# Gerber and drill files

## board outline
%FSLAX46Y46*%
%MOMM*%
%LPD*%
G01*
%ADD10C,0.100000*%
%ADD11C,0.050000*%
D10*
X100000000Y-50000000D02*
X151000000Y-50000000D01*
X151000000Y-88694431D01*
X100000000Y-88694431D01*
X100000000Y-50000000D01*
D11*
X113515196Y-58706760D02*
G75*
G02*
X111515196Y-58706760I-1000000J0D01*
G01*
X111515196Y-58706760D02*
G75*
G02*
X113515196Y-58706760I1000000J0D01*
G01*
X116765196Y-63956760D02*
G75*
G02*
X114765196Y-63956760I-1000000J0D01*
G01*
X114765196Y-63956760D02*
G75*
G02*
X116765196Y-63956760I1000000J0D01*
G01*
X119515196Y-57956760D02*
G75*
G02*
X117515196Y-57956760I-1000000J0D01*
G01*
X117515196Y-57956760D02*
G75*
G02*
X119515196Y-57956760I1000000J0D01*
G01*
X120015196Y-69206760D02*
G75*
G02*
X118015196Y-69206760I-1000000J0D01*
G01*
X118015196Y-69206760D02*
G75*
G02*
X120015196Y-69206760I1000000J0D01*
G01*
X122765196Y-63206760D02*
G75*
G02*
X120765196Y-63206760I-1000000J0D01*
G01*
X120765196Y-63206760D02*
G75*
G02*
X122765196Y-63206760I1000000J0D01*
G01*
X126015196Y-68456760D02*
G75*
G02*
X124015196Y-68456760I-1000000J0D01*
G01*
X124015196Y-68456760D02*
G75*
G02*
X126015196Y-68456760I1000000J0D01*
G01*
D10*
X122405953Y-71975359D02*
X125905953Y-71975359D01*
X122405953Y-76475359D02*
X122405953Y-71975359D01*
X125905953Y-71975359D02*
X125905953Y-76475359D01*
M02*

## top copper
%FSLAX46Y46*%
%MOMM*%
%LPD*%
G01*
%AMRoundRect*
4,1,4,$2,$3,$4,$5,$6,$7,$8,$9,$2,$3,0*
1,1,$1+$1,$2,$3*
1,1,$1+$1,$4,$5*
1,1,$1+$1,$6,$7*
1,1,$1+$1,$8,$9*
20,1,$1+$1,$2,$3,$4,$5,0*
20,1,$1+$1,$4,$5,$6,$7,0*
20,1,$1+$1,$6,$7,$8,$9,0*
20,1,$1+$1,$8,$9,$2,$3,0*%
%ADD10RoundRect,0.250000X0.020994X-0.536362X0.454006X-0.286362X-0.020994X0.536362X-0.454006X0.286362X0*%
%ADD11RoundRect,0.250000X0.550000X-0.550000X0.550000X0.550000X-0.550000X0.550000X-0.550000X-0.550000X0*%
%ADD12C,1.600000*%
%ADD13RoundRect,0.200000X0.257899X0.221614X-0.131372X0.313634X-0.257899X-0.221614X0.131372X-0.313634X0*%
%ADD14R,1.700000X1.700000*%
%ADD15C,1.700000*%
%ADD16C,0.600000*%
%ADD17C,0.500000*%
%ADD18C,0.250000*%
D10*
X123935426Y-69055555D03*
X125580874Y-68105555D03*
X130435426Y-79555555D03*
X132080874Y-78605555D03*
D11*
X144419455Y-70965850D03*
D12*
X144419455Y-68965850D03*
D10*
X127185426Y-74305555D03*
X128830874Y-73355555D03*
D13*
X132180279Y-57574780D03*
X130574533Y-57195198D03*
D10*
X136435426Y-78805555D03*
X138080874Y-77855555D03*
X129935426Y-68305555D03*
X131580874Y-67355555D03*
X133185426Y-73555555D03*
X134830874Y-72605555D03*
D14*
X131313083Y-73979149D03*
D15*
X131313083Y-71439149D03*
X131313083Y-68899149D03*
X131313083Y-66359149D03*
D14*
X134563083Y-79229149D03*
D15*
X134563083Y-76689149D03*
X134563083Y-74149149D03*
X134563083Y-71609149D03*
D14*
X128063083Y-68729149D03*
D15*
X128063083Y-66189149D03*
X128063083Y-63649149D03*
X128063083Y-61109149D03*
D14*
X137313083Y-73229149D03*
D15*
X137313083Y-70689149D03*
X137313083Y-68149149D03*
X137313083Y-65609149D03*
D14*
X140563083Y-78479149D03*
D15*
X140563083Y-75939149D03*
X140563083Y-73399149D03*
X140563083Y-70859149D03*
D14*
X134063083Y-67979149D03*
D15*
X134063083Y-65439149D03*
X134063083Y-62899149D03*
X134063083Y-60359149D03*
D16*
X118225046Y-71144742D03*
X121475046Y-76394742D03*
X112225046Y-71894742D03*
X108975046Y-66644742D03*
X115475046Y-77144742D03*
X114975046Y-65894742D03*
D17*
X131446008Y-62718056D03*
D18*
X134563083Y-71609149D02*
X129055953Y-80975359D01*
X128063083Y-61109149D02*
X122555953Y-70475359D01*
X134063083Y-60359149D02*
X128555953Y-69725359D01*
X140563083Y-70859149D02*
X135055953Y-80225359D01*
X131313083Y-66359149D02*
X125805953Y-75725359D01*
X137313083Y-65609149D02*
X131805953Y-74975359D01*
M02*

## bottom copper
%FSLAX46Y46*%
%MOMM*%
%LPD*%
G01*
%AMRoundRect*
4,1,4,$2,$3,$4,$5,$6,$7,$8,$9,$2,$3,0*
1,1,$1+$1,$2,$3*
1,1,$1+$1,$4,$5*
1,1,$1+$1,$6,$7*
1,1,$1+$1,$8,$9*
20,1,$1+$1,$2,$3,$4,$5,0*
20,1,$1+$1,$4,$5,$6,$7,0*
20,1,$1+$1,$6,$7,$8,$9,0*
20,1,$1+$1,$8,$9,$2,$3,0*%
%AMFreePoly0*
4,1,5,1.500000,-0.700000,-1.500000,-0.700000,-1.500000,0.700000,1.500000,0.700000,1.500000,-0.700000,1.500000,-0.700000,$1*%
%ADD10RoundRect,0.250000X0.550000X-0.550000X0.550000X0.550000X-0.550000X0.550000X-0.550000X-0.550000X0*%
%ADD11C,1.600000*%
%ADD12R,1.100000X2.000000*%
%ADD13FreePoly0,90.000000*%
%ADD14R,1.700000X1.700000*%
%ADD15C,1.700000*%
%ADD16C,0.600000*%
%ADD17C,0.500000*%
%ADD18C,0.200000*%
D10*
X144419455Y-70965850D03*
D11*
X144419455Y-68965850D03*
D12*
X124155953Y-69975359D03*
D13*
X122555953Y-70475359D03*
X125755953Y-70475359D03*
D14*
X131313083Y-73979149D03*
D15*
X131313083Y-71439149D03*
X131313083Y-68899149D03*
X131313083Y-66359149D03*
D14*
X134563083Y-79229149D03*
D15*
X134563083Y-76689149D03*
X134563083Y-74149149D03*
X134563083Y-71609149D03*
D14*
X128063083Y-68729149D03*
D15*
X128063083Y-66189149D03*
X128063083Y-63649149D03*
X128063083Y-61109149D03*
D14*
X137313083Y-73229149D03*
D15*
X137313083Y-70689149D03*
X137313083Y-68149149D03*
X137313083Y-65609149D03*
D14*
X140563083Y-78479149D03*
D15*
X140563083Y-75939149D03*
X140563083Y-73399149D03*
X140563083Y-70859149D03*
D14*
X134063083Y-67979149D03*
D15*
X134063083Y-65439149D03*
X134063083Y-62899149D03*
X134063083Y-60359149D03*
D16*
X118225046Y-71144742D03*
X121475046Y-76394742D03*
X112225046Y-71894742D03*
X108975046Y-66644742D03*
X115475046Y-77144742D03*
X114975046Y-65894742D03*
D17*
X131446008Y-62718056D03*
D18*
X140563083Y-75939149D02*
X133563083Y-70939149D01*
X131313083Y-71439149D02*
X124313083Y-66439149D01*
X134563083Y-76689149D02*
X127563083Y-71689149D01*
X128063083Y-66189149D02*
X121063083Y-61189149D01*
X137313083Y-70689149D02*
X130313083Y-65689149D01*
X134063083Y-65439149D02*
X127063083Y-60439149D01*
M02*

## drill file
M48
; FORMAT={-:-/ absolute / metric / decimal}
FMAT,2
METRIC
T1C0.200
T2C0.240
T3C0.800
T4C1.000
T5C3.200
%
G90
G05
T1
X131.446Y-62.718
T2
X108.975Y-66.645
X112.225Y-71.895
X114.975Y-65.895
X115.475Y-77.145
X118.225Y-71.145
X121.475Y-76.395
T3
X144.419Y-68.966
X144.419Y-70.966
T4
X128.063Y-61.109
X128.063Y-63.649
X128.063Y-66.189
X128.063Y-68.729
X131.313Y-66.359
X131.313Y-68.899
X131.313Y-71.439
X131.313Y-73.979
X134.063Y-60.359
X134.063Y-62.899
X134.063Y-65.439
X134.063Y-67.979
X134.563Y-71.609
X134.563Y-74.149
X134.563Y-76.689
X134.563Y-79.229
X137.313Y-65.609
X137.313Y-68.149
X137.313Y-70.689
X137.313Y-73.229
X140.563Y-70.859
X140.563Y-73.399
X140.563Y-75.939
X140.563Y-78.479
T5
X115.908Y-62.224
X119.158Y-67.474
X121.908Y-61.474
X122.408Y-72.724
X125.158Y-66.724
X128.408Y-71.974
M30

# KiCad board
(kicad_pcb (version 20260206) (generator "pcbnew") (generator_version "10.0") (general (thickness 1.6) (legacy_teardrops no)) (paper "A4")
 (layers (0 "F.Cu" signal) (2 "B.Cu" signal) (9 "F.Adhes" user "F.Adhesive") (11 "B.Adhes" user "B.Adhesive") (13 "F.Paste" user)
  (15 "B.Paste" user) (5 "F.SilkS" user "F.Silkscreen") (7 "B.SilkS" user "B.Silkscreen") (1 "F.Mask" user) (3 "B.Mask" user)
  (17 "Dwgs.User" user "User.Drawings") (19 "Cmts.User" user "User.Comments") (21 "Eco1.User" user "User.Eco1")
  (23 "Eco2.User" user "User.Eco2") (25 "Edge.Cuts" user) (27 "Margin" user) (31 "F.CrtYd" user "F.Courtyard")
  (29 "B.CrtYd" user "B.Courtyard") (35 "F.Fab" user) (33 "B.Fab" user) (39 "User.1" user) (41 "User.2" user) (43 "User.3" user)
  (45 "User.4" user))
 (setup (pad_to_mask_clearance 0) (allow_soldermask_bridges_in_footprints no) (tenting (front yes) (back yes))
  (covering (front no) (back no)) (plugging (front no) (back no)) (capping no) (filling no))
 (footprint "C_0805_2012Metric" (layer "F.Cu") (at 124.75815 68.580555 30)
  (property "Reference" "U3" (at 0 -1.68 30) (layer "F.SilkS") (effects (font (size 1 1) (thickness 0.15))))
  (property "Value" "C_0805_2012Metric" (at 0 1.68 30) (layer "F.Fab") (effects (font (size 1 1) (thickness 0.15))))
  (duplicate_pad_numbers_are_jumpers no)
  (pad "1" smd roundrect (at -0.95 0 30) (size 1 1.45) (layers "F.Cu" "F.Mask" "F.Paste") (roundrect_rratio 0.25) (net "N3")
   (clearance 0.35))
  (pad "2" smd roundrect (at 0.95 0 30) (size 1 1.45) (layers "F.Cu" "F.Mask" "F.Paste") (roundrect_rratio 0.25)))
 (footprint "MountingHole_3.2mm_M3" (layer "F.Cu") (at 119.158484 67.474067 45)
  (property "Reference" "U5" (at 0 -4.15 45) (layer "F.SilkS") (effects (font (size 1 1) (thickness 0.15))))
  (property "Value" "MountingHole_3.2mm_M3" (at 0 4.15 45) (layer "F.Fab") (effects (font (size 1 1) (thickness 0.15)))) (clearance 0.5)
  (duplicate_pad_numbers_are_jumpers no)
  (pad "" np_thru_hole circle (at 0 0 45) (size 3.2 3.2) (drill 3.2) (layers "*.Cu" "*.Mask")))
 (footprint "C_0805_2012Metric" (layer "F.Cu") (at 131.25815 79.080555 30)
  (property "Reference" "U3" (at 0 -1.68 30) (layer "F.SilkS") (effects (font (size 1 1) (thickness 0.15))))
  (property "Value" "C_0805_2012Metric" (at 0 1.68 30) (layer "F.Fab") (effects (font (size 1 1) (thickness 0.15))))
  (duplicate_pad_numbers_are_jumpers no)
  (pad "1" smd roundrect (at -0.95 0 30) (size 1 1.45) (layers "F.Cu" "F.Mask" "F.Paste") (roundrect_rratio 0.25) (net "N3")
   (clearance 0.35))
  (pad "2" smd roundrect (at 0.95 0 30) (size 1 1.45) (layers "F.Cu" "F.Mask" "F.Paste") (roundrect_rratio 0.25)))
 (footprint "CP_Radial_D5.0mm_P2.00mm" (layer "F.Cu") (at 144.419455 70.96585 90)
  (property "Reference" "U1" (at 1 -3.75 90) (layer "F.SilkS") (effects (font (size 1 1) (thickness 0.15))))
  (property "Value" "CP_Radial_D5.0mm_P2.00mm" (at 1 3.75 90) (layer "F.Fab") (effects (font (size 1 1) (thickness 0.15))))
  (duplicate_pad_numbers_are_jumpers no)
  (pad "1" thru_hole roundrect (at 0 0 90) (size 1.6 1.6) (drill 0.8) (layers "*.Cu" "*.Mask") (remove_unused_layers no)
   (roundrect_rratio 0.15625) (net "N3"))
  (pad "2" thru_hole circle (at 2 0 90) (size 1.6 1.6) (drill 0.8) (layers "*.Cu" "*.Mask") (remove_unused_layers no) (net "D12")))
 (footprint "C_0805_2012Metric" (layer "F.Cu") (at 128.00815 73.830555 30)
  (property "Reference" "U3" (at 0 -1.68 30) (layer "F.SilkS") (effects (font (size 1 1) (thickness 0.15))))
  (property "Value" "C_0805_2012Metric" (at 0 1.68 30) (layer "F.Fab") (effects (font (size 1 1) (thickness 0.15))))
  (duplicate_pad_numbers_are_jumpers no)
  (pad "1" smd roundrect (at -0.95 0 30) (size 1 1.45) (layers "F.Cu" "F.Mask" "F.Paste") (roundrect_rratio 0.25) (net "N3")
   (clearance 0.35))
  (pad "2" smd roundrect (at 0.95 0 30) (size 1 1.45) (layers "F.Cu" "F.Mask" "F.Paste") (roundrect_rratio 0.25)))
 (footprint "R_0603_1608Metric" (layer "F.Cu") (at 131.377406 57.384989 166.7)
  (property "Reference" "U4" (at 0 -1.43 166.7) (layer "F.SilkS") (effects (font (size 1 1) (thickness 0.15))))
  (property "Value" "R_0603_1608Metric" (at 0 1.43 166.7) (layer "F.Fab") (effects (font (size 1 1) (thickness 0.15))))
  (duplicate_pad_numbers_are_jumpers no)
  (pad "1" smd roundrect (at -0.825 0 166.7) (size 0.8 0.95) (layers "F.Cu" "F.Mask" "F.Paste") (roundrect_rratio 0.25) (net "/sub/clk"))
  (pad "2" smd roundrect (at 0.825 0 166.7) (size 0.8 0.95) (layers "F.Cu" "F.Mask" "F.Paste") (roundrect_rratio 0.25) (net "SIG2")))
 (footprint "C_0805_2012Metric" (layer "F.Cu") (at 137.25815 78.330555 30)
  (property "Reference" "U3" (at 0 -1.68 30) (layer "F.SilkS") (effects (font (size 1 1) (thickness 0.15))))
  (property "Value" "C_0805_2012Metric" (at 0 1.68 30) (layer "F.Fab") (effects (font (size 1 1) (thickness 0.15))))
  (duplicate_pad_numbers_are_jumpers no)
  (pad "1" smd roundrect (at -0.95 0 30) (size 1 1.45) (layers "F.Cu" "F.Mask" "F.Paste") (roundrect_rratio 0.25) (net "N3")
   (clearance 0.35))
  (pad "2" smd roundrect (at 0.95 0 30) (size 1 1.45) (layers "F.Cu" "F.Mask" "F.Paste") (roundrect_rratio 0.25)))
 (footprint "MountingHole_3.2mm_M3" (layer "F.Cu") (at 115.908484 62.224067 45)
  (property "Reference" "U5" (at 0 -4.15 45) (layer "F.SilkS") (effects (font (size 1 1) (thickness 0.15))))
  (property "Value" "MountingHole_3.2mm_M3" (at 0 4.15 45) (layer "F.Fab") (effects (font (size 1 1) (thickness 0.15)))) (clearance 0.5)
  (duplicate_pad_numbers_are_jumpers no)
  (pad "" np_thru_hole circle (at 0 0 45) (size 3.2 3.2) (drill 3.2) (layers "*.Cu" "*.Mask")))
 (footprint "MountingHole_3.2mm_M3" (layer "F.Cu") (at 122.408484 72.724067 45)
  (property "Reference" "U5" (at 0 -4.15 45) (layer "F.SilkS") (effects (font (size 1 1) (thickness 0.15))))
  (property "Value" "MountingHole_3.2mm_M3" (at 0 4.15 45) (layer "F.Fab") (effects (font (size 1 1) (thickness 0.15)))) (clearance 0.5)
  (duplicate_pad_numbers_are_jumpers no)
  (pad "" np_thru_hole circle (at 0 0 45) (size 3.2 3.2) (drill 3.2) (layers "*.Cu" "*.Mask")))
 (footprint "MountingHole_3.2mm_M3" (layer "F.Cu") (at 125.158484 66.724067 45)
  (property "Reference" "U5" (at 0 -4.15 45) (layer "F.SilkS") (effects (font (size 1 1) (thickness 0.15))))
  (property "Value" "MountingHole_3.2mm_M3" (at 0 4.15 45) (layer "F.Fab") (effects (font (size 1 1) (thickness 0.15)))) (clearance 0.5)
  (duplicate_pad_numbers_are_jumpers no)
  (pad "" np_thru_hole circle (at 0 0 45) (size 3.2 3.2) (drill 3.2) (layers "*.Cu" "*.Mask")))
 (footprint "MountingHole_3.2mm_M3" (layer "F.Cu") (at 121.908484 61.474067 45)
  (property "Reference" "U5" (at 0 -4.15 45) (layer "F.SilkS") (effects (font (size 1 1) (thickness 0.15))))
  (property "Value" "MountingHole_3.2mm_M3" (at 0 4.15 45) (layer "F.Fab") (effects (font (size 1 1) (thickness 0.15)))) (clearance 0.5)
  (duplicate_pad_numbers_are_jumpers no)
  (pad "" np_thru_hole circle (at 0 0 45) (size 3.2 3.2) (drill 3.2) (layers "*.Cu" "*.Mask")))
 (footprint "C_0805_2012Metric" (layer "F.Cu") (at 130.75815 67.830555 30)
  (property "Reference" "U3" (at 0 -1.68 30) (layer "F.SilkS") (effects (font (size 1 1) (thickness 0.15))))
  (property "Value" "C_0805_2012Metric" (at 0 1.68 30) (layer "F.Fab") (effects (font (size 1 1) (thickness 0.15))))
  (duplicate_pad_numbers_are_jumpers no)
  (pad "1" smd roundrect (at -0.95 0 30) (size 1 1.45) (layers "F.Cu" "F.Mask" "F.Paste") (roundrect_rratio 0.25) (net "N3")
   (clearance 0.35))
  (pad "2" smd roundrect (at 0.95 0 30) (size 1 1.45) (layers "F.Cu" "F.Mask" "F.Paste") (roundrect_rratio 0.25)))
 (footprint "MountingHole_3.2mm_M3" (layer "F.Cu") (at 128.408484 71.974067 45)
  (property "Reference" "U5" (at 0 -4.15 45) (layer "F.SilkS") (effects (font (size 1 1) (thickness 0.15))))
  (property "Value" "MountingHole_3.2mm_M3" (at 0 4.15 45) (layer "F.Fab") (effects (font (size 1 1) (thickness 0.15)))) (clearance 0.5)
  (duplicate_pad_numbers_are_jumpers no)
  (pad "" np_thru_hole circle (at 0 0 45) (size 3.2 3.2) (drill 3.2) (layers "*.Cu" "*.Mask")))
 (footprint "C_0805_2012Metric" (layer "F.Cu") (at 134.00815 73.080555 30)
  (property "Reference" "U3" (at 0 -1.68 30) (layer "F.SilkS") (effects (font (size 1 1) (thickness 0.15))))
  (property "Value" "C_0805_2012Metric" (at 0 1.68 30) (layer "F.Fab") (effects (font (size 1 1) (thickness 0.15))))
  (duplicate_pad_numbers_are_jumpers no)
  (pad "1" smd roundrect (at -0.95 0 30) (size 1 1.45) (layers "F.Cu" "F.Mask" "F.Paste") (roundrect_rratio 0.25) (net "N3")
   (clearance 0.35))
  (pad "2" smd roundrect (at 0.95 0 30) (size 1 1.45) (layers "F.Cu" "F.Mask" "F.Paste") (roundrect_rratio 0.25)))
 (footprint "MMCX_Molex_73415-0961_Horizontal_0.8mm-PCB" (layer "B.Cu") (at 124.155953 72.725359 90)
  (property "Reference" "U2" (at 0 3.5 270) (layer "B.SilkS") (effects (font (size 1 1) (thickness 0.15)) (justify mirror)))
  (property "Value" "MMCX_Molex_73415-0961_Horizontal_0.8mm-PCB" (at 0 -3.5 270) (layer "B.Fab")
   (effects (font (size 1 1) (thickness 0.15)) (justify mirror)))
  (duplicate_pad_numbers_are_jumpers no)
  (fp_line (start 0.75 -1.75) (end 0.75 1.75) (stroke (width 0.1) (type solid)) (layer "Edge.Cuts"))
  (fp_line (start -3.75 -1.75) (end 0.75 -1.75) (stroke (width 0.1) (type solid)) (layer "Edge.Cuts"))
  (fp_line (start 0.75 1.75) (end -3.75 1.75) (stroke (width 0.1) (type solid)) (layer "Edge.Cuts"))
  (pad "1" smd rect (at 2.75 0 90) (size 2 1.1) (layers "B.Cu" "B.Mask" "B.Paste") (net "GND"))
  (pad "2" smd custom (at 2.25 -1.6 90) (size 3 1.4) (layers "B.Cu" "B.Mask" "B.Paste") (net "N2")
   (options (clearance outline) (anchor rect)) (primitives))
  (pad "2" smd custom (at 2.25 1.6 90) (size 3 1.4) (layers "B.Cu" "B.Mask" "B.Paste") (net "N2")
   (options (clearance outline) (anchor rect)) (primitives)))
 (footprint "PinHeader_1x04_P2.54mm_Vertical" (layer "B.Cu") (at 131.313083 73.979149)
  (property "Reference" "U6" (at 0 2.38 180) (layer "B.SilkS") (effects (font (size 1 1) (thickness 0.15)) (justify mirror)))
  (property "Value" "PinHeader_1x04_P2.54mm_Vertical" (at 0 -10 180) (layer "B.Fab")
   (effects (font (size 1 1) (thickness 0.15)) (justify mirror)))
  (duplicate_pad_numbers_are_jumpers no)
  (pad "1" thru_hole rect (at 0 0) (size 1.7 1.7) (drill 1) (layers "*.Cu" "*.Mask") (remove_unused_layers no) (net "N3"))
  (pad "2" thru_hole circle (at 0 -2.54) (size 1.7 1.7) (drill 1) (layers "*.Cu" "*.Mask") (remove_unused_layers no) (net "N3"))
  (pad "3" thru_hole circle (at 0 -5.08) (size 1.7 1.7) (drill 1) (layers "*.Cu" "*.Mask") (remove_unused_layers no) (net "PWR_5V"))
  (pad "4" thru_hole circle (at 0 -7.62) (size 1.7 1.7) (drill 1) (layers "*.Cu" "*.Mask") (remove_unused_layers no)))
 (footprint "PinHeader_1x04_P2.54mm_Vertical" (layer "B.Cu") (at 134.563083 79.229149)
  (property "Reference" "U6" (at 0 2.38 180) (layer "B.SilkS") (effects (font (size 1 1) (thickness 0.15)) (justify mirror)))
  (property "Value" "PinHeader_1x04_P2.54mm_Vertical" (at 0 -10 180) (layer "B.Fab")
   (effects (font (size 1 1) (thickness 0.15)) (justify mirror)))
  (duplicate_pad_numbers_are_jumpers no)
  (pad "1" thru_hole rect (at 0 0) (size 1.7 1.7) (drill 1) (layers "*.Cu" "*.Mask") (remove_unused_layers no) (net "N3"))
  (pad "2" thru_hole circle (at 0 -2.54) (size 1.7 1.7) (drill 1) (layers "*.Cu" "*.Mask") (remove_unused_layers no) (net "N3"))
  (pad "3" thru_hole circle (at 0 -5.08) (size 1.7 1.7) (drill 1) (layers "*.Cu" "*.Mask") (remove_unused_layers no) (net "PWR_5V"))
  (pad "4" thru_hole circle (at 0 -7.62) (size 1.7 1.7) (drill 1) (layers "*.Cu" "*.Mask") (remove_unused_layers no)))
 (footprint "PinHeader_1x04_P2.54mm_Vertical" (layer "B.Cu") (at 128.063083 68.729149)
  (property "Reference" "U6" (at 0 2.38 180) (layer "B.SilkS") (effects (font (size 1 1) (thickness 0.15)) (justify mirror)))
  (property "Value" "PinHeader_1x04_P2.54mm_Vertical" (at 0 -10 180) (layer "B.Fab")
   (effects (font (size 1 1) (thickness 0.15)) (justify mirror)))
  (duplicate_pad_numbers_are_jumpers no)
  (pad "1" thru_hole rect (at 0 0) (size 1.7 1.7) (drill 1) (layers "*.Cu" "*.Mask") (remove_unused_layers no) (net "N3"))
  (pad "2" thru_hole circle (at 0 -2.54) (size 1.7 1.7) (drill 1) (layers "*.Cu" "*.Mask") (remove_unused_layers no) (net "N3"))
  (pad "3" thru_hole circle (at 0 -5.08) (size 1.7 1.7) (drill 1) (layers "*.Cu" "*.Mask") (remove_unused_layers no) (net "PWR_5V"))
  (pad "4" thru_hole circle (at 0 -7.62) (size 1.7 1.7) (drill 1) (layers "*.Cu" "*.Mask") (remove_unused_layers no)))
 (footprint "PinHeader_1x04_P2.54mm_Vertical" (layer "B.Cu") (at 137.313083 73.229149)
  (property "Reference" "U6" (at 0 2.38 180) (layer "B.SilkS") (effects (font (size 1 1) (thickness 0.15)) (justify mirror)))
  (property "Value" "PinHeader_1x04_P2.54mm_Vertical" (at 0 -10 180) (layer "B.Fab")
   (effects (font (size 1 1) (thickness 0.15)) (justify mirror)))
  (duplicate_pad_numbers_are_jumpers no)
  (pad "1" thru_hole rect (at 0 0) (size 1.7 1.7) (drill 1) (layers "*.Cu" "*.Mask") (remove_unused_layers no) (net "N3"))
  (pad "2" thru_hole circle (at 0 -2.54) (size 1.7 1.7) (drill 1) (layers "*.Cu" "*.Mask") (remove_unused_layers no) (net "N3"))
  (pad "3" thru_hole circle (at 0 -5.08) (size 1.7 1.7) (drill 1) (layers "*.Cu" "*.Mask") (remove_unused_layers no) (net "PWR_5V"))
  (pad "4" thru_hole circle (at 0 -7.62) (size 1.7 1.7) (drill 1) (layers "*.Cu" "*.Mask") (remove_unused_layers no)))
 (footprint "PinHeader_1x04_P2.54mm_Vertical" (layer "B.Cu") (at 140.563083 78.479149)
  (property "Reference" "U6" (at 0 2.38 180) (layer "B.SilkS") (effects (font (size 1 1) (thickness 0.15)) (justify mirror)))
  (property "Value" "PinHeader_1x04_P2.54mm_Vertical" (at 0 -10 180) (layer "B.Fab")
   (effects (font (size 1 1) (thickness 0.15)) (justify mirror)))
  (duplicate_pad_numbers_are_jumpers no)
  (pad "1" thru_hole rect (at 0 0) (size 1.7 1.7) (drill 1) (layers "*.Cu" "*.Mask") (remove_unused_layers no) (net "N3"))
  (pad "2" thru_hole circle (at 0 -2.54) (size 1.7 1.7) (drill 1) (layers "*.Cu" "*.Mask") (remove_unused_layers no) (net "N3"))
  (pad "3" thru_hole circle (at 0 -5.08) (size 1.7 1.7) (drill 1) (layers "*.Cu" "*.Mask") (remove_unused_layers no) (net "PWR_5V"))
  (pad "4" thru_hole circle (at 0 -7.62) (size 1.7 1.7) (drill 1) (layers "*.Cu" "*.Mask") (remove_unused_layers no)))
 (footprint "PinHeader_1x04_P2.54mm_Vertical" (layer "B.Cu") (at 134.063083 67.979149)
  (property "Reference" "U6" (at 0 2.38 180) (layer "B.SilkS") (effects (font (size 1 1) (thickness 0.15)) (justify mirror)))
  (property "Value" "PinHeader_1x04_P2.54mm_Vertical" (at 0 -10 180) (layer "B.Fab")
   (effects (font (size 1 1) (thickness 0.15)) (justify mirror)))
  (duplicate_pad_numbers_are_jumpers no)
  (pad "1" thru_hole rect (at 0 0) (size 1.7 1.7) (drill 1) (layers "*.Cu" "*.Mask") (remove_unused_layers no) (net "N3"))
  (pad "2" thru_hole circle (at 0 -2.54) (size 1.7 1.7) (drill 1) (layers "*.Cu" "*.Mask") (remove_unused_layers no) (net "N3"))
  (pad "3" thru_hole circle (at 0 -5.08) (size 1.7 1.7) (drill 1) (layers "*.Cu" "*.Mask") (remove_unused_layers no) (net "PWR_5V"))
  (pad "4" thru_hole circle (at 0 -7.62) (size 1.7 1.7) (drill 1) (layers "*.Cu" "*.Mask") (remove_unused_layers no)))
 (gr_rect (start 100 50) (end 151 88.694431) (stroke (width 0.1) (type default)) (fill no) (layer "Edge.Cuts"))
 (gr_circle (center 112.515196 58.70676) (end 113.515196 58.70676) (stroke (width 0.05) (type default)) (fill no) (layer "Edge.Cuts"))
 (gr_circle (center 115.765196 63.95676) (end 116.765196 63.95676) (stroke (width 0.05) (type default)) (fill no) (layer "Edge.Cuts"))
 (gr_circle (center 118.515196 57.95676) (end 119.515196 57.95676) (stroke (width 0.05) (type default)) (fill no) (layer "Edge.Cuts"))
 (gr_circle (center 119.015196 69.20676) (end 120.015196 69.20676) (stroke (width 0.05) (type default)) (fill no) (layer "Edge.Cuts"))
 (gr_circle (center 121.765196 63.20676) (end 122.765196 63.20676) (stroke (width 0.05) (type default)) (fill no) (layer "Edge.Cuts"))
 (gr_circle (center 125.015196 68.45676) (end 126.015196 68.45676) (stroke (width 0.05) (type default)) (fill no) (layer "Edge.Cuts"))
 (segment (start 134.563083 71.609149) (end 129.055953 80.975359) (width 0.25) (layer "F.Cu") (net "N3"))
 (segment (start 128.063083 61.109149) (end 122.555953 70.475359) (width 0.25) (layer "F.Cu") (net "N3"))
 (segment (start 134.063083 60.359149) (end 128.555953 69.725359) (width 0.25) (layer "F.Cu") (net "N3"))
 (segment (start 140.563083 70.859149) (end 135.055953 80.225359) (width 0.25) (layer "F.Cu") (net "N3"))
 (segment (start 131.313083 66.359149) (end 125.805953 75.725359) (width 0.25) (layer "F.Cu") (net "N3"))
 (segment (start 137.313083 65.609149) (end 131.805953 74.975359) (width 0.25) (layer "F.Cu") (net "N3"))
 (segment (start 140.563083 75.939149) (end 133.563083 70.939149) (width 0.2) (layer "B.Cu") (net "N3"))
 (segment (start 131.313083 71.439149) (end 124.313083 66.439149) (width 0.2) (layer "B.Cu") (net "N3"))
 (segment (start 134.563083 76.689149) (end 127.563083 71.689149) (width 0.2) (layer "B.Cu") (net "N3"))
 (segment (start 128.063083 66.189149) (end 121.063083 61.189149) (width 0.2) (layer "B.Cu") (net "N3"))
 (segment (start 137.313083 70.689149) (end 130.313083 65.689149) (width 0.2) (layer "B.Cu") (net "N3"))
 (segment (start 134.063083 65.439149) (end 127.063083 60.439149) (width 0.2) (layer "B.Cu") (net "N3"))
 (via (at 118.225046 71.144742) (size 0.6) (drill 0.24) (layers "F.Cu" "B.Cu") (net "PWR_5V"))
 (via (at 121.475046 76.394742) (size 0.6) (drill 0.24) (layers "F.Cu" "B.Cu") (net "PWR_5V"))
 (via (at 112.225046 71.894742) (size 0.6) (drill 0.24) (layers "F.Cu" "B.Cu") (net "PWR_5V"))
 (via (at 108.975046 66.644742) (size 0.6) (drill 0.24) (layers "F.Cu" "B.Cu") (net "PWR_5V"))
 (via (at 115.475046 77.144742) (size 0.6) (drill 0.24) (layers "F.Cu" "B.Cu") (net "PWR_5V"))
 (via (at 114.975046 65.894742) (size 0.6) (drill 0.24) (layers "F.Cu" "B.Cu") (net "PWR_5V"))
 (via (at 131.446008 62.718056) (size 0.5) (drill 0.2) (layers "F.Cu" "B.Cu") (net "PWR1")))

